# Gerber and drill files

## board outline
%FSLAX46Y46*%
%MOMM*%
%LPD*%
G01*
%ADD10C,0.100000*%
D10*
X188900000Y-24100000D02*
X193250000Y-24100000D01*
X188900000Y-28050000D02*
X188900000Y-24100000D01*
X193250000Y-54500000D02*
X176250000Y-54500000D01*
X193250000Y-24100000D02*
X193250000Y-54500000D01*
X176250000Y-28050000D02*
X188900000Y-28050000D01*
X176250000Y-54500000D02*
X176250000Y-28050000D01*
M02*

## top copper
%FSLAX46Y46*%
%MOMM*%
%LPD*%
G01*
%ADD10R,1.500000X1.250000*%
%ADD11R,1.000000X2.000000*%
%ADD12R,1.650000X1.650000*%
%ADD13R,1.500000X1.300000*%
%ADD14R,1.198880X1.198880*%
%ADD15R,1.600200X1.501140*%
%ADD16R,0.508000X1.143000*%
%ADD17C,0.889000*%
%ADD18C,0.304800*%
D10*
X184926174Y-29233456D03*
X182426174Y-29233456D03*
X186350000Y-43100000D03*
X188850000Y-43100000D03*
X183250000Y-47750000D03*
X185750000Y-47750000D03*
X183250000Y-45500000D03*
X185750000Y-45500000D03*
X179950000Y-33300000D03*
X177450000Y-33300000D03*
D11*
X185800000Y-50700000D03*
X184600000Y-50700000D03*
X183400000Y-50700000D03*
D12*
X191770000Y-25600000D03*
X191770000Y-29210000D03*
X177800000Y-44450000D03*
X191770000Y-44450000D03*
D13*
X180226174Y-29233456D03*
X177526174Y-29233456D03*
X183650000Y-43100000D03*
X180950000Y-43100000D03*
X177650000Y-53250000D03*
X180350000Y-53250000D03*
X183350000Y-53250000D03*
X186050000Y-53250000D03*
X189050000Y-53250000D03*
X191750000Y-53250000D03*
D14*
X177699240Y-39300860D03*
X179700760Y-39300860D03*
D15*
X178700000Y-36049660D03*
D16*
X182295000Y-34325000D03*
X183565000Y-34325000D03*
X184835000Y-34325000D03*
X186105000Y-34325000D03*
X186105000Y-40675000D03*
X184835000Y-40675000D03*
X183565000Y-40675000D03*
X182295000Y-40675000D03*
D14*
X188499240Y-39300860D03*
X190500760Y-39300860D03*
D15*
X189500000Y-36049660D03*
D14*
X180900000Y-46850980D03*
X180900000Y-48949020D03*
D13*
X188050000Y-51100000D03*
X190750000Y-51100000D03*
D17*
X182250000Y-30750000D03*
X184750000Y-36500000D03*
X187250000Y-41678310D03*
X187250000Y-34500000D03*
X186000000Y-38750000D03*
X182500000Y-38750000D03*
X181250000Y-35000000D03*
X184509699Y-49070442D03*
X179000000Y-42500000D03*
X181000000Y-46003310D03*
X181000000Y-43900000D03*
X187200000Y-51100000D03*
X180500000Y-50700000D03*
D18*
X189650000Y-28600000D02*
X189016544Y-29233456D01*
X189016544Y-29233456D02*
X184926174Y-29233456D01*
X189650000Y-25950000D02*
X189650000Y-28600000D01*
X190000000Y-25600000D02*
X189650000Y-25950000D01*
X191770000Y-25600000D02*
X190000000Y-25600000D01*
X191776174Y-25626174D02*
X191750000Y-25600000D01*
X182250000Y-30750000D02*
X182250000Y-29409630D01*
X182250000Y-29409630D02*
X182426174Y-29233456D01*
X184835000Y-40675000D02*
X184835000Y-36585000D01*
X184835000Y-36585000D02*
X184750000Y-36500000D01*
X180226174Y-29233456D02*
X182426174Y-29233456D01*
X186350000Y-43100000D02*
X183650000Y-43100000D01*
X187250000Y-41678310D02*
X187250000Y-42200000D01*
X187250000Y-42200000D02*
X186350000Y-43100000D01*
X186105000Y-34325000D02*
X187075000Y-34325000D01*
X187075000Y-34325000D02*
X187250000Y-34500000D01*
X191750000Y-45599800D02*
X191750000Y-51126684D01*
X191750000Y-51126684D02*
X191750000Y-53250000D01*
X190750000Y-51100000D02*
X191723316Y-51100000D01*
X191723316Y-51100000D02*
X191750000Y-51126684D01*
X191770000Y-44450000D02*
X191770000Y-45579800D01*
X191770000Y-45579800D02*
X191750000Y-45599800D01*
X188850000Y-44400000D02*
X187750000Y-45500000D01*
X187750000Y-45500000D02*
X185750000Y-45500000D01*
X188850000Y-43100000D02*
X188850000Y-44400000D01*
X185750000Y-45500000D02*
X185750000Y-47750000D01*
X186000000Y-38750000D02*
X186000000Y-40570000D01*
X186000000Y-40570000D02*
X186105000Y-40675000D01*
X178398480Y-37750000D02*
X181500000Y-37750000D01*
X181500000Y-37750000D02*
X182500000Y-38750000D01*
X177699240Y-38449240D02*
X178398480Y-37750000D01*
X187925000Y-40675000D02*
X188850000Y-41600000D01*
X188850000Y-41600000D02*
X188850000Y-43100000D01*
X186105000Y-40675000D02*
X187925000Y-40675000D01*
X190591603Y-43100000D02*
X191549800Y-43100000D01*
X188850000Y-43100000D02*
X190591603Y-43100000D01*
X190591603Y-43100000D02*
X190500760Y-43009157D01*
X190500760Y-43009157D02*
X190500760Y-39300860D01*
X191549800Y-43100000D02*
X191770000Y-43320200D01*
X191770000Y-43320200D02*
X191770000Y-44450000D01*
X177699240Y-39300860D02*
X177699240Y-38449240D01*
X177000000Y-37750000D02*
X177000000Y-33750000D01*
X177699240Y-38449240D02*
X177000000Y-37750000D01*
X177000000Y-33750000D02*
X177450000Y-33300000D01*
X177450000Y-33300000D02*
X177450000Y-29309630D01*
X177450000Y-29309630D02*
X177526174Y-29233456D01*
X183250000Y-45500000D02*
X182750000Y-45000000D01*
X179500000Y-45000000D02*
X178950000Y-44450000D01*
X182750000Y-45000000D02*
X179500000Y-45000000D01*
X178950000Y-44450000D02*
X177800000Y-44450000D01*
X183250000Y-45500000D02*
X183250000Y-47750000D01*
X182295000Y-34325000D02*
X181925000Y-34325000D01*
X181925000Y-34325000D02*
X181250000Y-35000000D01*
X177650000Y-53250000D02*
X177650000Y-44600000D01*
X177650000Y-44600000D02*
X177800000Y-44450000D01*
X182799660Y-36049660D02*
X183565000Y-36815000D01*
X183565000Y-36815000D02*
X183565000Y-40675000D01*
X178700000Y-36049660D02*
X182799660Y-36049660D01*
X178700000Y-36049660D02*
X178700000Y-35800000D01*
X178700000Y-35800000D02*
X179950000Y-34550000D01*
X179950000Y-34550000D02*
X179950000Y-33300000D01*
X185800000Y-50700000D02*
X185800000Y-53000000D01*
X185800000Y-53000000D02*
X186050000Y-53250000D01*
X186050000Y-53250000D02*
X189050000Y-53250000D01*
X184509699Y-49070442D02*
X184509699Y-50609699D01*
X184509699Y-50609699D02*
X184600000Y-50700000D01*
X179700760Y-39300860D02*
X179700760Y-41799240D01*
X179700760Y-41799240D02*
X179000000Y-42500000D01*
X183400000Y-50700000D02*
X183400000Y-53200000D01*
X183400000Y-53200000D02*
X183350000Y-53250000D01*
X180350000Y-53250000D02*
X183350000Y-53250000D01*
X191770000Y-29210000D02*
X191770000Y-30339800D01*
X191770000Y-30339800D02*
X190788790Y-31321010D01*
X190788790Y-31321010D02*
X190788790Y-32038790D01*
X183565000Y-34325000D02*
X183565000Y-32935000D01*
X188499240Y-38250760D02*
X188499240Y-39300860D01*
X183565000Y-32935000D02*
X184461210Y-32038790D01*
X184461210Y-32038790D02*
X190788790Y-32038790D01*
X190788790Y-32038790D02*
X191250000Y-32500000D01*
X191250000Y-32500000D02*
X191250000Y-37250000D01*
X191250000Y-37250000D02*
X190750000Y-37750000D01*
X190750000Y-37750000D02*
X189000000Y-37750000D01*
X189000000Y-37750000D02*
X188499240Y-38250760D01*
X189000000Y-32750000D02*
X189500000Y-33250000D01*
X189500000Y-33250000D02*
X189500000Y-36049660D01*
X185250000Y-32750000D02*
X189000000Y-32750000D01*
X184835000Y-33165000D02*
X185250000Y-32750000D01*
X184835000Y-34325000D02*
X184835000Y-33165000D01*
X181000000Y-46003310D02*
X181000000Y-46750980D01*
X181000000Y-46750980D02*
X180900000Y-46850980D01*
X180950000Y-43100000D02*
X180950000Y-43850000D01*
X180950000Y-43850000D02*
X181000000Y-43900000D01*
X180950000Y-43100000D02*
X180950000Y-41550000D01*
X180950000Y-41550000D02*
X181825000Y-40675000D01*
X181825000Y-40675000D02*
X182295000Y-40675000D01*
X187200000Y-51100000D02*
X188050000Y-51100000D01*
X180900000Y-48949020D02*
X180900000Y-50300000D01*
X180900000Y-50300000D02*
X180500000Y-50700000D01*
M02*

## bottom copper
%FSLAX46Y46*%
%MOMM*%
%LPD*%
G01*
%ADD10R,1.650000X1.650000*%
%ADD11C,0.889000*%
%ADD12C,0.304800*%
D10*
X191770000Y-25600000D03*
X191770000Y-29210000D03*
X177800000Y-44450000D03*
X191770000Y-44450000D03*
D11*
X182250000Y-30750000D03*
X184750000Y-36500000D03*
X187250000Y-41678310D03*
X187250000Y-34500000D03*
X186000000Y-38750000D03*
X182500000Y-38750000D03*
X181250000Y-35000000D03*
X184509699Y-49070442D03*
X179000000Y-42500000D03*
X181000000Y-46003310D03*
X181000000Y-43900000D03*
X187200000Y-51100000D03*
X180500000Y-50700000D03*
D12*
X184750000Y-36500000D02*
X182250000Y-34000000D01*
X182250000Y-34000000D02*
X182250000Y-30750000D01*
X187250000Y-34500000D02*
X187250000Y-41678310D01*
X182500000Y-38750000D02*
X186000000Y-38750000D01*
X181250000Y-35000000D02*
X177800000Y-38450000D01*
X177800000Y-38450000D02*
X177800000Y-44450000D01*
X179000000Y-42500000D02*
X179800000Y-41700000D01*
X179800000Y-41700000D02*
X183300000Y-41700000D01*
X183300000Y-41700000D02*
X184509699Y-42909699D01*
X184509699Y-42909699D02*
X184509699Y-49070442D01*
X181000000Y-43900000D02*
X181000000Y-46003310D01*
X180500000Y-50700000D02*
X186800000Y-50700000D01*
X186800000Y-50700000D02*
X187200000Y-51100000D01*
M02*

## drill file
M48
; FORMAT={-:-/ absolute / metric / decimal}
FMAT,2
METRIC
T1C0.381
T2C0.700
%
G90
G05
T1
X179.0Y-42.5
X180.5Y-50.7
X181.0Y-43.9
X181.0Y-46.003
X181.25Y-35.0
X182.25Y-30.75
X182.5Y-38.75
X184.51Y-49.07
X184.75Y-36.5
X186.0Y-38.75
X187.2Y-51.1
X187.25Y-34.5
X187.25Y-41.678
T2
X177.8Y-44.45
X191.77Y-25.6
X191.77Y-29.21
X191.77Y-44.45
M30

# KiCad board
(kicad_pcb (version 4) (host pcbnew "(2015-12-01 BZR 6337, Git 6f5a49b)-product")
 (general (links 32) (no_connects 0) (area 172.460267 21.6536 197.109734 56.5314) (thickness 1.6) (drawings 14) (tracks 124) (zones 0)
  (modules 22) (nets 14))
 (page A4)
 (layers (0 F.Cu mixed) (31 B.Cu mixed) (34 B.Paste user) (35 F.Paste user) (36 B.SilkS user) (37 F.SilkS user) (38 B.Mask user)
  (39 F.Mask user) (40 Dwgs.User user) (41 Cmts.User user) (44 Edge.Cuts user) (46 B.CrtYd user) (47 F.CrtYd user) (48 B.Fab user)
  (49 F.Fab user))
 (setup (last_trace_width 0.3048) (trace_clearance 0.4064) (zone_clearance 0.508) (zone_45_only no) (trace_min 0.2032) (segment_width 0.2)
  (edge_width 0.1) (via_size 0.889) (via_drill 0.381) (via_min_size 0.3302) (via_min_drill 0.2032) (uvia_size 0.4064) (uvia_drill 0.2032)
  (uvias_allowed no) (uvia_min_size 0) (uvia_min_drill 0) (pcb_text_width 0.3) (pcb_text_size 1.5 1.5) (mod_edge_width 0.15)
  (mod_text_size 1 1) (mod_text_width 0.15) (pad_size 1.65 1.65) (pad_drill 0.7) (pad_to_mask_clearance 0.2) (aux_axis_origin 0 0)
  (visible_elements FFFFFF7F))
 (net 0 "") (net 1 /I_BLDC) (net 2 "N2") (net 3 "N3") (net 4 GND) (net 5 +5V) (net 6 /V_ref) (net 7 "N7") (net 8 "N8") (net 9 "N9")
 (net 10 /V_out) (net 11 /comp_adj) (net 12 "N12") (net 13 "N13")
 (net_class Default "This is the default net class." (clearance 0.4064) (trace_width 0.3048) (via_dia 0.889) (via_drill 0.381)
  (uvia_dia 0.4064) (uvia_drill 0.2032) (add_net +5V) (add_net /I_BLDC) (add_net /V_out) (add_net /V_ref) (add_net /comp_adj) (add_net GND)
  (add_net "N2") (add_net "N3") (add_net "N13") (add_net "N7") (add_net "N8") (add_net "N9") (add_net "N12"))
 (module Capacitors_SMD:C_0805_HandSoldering (layer F.Cu) (at 183.676174 29.233456 180)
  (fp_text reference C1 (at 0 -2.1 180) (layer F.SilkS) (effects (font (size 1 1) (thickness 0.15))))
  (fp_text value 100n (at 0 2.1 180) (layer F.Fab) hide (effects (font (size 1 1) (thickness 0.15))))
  (pad 1 smd rect (at -1.25 0 180) (size 1.5 1.25) (layers F.Cu F.Paste F.Mask) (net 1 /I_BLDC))
  (pad 2 smd rect (at 1.25 0 180) (size 1.5 1.25) (layers F.Cu F.Paste F.Mask) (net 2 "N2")))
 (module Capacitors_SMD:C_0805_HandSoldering (layer F.Cu) (at 187.6 43.1)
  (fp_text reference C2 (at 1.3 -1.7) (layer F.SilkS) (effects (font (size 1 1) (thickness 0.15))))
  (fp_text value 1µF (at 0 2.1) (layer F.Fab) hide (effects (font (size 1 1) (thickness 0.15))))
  (pad 1 smd rect (at -1.25 0) (size 1.5 1.25) (layers F.Cu F.Paste F.Mask) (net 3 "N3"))
  (pad 2 smd rect (at 1.25 0) (size 1.5 1.25) (layers F.Cu F.Paste F.Mask) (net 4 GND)))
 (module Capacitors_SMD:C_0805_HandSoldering (layer F.Cu) (at 184.5 47.75)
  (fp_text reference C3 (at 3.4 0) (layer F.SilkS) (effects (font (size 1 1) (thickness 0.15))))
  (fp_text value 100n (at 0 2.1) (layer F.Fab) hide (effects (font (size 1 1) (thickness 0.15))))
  (pad 1 smd rect (at -1.25 0) (size 1.5 1.25) (layers F.Cu F.Paste F.Mask) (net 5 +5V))
  (pad 2 smd rect (at 1.25 0) (size 1.5 1.25) (layers F.Cu F.Paste F.Mask) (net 4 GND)))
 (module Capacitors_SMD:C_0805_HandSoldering (layer F.Cu) (at 184.5 45.5)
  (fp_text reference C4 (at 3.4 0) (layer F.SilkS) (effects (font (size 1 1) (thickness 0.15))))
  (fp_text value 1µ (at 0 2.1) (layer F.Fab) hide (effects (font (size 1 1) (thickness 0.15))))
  (pad 1 smd rect (at -1.25 0) (size 1.5 1.25) (layers F.Cu F.Paste F.Mask) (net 5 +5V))
  (pad 2 smd rect (at 1.25 0) (size 1.5 1.25) (layers F.Cu F.Paste F.Mask) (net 4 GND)))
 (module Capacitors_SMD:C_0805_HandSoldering (layer F.Cu) (at 178.7 33.3 180)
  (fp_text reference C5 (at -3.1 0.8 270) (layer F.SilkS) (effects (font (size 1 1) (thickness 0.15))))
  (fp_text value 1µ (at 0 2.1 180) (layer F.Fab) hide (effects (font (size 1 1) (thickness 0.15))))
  (pad 1 smd rect (at -1.25 0 180) (size 1.5 1.25) (layers F.Cu F.Paste F.Mask) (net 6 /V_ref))
  (pad 2 smd rect (at 1.25 0 180) (size 1.5 1.25) (layers F.Cu F.Paste F.Mask) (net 4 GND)))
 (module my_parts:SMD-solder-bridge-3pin (layer F.Cu) (at 184.6 50.7 180) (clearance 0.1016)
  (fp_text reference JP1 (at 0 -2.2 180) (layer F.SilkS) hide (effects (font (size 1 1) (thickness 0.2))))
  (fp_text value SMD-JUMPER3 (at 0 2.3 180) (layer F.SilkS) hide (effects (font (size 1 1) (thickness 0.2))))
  (pad 1 smd rect (at -1.2 0 180) (size 1 2) (layers F.Cu F.Mask) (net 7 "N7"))
  (pad 2 smd rect (at 0 0 180) (size 1 2) (layers F.Cu F.Mask) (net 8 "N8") (solder_mask_margin 0.3))
  (pad 3 smd rect (at 1.2 0 180) (size 1 2) (layers F.Cu F.Mask) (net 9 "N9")))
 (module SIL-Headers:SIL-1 (layer F.Cu) (at 191.77 25.6)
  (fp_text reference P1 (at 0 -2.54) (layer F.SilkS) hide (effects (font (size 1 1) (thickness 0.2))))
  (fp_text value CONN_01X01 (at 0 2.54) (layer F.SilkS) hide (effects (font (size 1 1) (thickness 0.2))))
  (pad 1 thru_hole rect (at 0 0) (size 1.65 1.65) (drill 0.7) (layers *.Cu *.Mask) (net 1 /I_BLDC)))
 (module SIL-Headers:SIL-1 (layer F.Cu) (at 191.77 29.21)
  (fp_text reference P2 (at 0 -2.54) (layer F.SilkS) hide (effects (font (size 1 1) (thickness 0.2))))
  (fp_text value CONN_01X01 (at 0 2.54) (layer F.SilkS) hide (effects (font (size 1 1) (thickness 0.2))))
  (pad 1 thru_hole rect (at 0 0) (size 1.65 1.65) (drill 0.7) (layers *.Cu *.Mask) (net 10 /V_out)))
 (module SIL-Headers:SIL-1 (layer F.Cu) (at 177.8 44.45)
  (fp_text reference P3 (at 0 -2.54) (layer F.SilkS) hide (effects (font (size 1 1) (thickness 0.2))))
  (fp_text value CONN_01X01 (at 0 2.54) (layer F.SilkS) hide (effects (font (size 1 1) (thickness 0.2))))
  (pad 1 thru_hole rect (at 0 0) (size 1.65 1.65) (drill 0.7) (layers *.Cu *.Mask) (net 5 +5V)))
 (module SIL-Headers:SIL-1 (layer F.Cu) (at 191.77 44.45)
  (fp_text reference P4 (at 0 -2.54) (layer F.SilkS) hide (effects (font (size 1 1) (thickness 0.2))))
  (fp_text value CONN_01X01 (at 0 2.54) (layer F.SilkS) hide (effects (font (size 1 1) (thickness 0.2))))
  (pad 1 thru_hole rect (at 0 0) (size 1.65 1.65) (drill 0.7) (layers *.Cu *.Mask) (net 4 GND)))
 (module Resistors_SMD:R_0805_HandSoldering (layer F.Cu) (at 178.876174 29.233456 180)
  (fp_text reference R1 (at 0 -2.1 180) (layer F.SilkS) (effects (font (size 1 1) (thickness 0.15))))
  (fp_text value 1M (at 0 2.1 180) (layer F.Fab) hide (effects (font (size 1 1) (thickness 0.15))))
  (pad 1 smd rect (at -1.35 0 180) (size 1.5 1.3) (layers F.Cu F.Paste F.Mask) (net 2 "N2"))
  (pad 2 smd rect (at 1.35 0 180) (size 1.5 1.3) (layers F.Cu F.Paste F.Mask) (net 4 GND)))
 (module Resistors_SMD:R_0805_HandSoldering (layer F.Cu) (at 182.3 43.1 180)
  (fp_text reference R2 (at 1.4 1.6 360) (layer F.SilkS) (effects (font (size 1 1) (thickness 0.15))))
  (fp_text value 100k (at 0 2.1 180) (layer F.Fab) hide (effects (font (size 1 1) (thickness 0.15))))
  (pad 1 smd rect (at -1.35 0 180) (size 1.5 1.3) (layers F.Cu F.Paste F.Mask) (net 3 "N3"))
  (pad 2 smd rect (at 1.35 0 180) (size 1.5 1.3) (layers F.Cu F.Paste F.Mask) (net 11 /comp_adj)))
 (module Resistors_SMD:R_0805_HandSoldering (layer F.Cu) (at 179 53.25)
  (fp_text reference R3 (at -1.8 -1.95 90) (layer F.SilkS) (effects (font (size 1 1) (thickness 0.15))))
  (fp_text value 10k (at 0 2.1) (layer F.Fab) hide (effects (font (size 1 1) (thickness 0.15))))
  (pad 1 smd rect (at -1.35 0) (size 1.5 1.3) (layers F.Cu F.Paste F.Mask) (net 5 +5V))
  (pad 2 smd rect (at 1.35 0) (size 1.5 1.3) (layers F.Cu F.Paste F.Mask) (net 9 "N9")))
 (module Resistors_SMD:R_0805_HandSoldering (layer F.Cu) (at 184.7 53.25)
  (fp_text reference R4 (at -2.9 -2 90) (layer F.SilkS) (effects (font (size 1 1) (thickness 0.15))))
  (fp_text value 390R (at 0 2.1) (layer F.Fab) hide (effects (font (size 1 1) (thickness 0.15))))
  (pad 1 smd rect (at -1.35 0) (size 1.5 1.3) (layers F.Cu F.Paste F.Mask) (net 9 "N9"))
  (pad 2 smd rect (at 1.35 0) (size 1.5 1.3) (layers F.Cu F.Paste F.Mask) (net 7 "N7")))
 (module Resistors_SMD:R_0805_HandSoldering (layer F.Cu) (at 190.4 53.25)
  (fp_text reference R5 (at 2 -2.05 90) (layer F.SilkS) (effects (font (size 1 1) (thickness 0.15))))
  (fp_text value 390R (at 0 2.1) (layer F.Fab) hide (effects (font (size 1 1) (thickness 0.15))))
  (pad 1 smd rect (at -1.35 0) (size 1.5 1.3) (layers F.Cu F.Paste F.Mask) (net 7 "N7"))
  (pad 2 smd rect (at 1.35 0) (size 1.5 1.3) (layers F.Cu F.Paste F.Mask) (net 4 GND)))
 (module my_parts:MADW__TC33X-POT (layer F.Cu) (at 178.7 37.5)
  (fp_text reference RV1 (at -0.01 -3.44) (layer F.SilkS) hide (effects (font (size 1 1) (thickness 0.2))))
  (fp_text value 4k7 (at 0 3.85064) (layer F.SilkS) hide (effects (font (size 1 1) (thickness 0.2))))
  (pad 1 smd rect (at -1.00076 1.80086) (size 1.19888 1.19888) (layers F.Cu F.Paste F.Mask) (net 4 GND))
  (pad 3 smd rect (at 1.00076 1.80086) (size 1.19888 1.19888) (layers F.Cu F.Paste F.Mask) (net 8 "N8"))
  (pad 2 smd rect (at 0 -1.45034) (size 1.6002 1.50114) (layers F.Cu F.Paste F.Mask) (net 6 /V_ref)))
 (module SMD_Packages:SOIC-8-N (layer F.Cu) (at 184.2 37.5)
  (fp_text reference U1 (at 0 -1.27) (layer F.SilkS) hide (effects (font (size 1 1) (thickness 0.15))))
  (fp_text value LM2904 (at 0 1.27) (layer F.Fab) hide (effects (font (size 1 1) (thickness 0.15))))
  (pad 8 smd rect (at -1.905 -3.175) (size 0.508 1.143) (layers F.Cu F.Paste F.Mask) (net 5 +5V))
  (pad 7 smd rect (at -0.635 -3.175) (size 0.508 1.143) (layers F.Cu F.Paste F.Mask) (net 10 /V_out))
  (pad 6 smd rect (at 0.635 -3.175) (size 0.508 1.143) (layers F.Cu F.Paste F.Mask) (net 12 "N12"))
  (pad 5 smd rect (at 1.905 -3.175) (size 0.508 1.143) (layers F.Cu F.Paste F.Mask) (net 3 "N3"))
  (pad 4 smd rect (at 1.905 3.175) (size 0.508 1.143) (layers F.Cu F.Paste F.Mask) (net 4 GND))
  (pad 3 smd rect (at 0.635 3.175) (size 0.508 1.143) (layers F.Cu F.Paste F.Mask) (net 2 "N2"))
  (pad 2 smd rect (at -0.635 3.175) (size 0.508 1.143) (layers F.Cu F.Paste F.Mask) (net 6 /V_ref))
  (pad 1 smd rect (at -1.905 3.175) (size 0.508 1.143) (layers F.Cu F.Paste F.Mask) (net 11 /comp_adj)))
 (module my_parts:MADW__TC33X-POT (layer F.Cu) (at 189.5 37.5)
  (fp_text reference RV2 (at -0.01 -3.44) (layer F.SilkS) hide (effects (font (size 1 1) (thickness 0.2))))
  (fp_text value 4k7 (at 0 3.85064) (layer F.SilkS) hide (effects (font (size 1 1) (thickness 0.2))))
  (pad 1 smd rect (at -1.00076 1.80086) (size 1.19888 1.19888) (layers F.Cu F.Paste F.Mask) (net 10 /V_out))
  (pad 3 smd rect (at 1.00076 1.80086) (size 1.19888 1.19888) (layers F.Cu F.Paste F.Mask) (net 4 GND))
  (pad 2 smd rect (at 0 -1.45034) (size 1.6002 1.50114) (layers F.Cu F.Paste F.Mask) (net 12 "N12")))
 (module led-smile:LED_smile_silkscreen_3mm (layer F.Cu) (at 186.85 31.85)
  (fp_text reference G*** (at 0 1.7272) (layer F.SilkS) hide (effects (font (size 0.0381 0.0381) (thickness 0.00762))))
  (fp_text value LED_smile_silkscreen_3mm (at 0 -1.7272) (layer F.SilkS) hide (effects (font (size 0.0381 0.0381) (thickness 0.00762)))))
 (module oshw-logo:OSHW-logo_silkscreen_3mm (layer F.Cu) (at 191.7 41.45)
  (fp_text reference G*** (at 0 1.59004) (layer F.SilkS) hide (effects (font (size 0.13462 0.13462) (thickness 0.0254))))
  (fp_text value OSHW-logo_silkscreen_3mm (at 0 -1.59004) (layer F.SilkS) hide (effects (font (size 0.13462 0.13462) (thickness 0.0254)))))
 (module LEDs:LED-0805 (layer F.Cu) (at 180.9 47.9 90)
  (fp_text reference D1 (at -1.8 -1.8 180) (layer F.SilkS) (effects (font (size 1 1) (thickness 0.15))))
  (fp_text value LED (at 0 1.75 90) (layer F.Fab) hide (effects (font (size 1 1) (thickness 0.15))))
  (pad 2 smd rect (at 1.04902 0 270) (size 1.19888 1.19888) (layers F.Cu F.Paste F.Mask) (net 11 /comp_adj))
  (pad 1 smd rect (at -1.04902 0 270) (size 1.19888 1.19888) (layers F.Cu F.Paste F.Mask) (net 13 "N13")))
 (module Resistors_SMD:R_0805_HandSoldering (layer F.Cu) (at 189.4 51.1)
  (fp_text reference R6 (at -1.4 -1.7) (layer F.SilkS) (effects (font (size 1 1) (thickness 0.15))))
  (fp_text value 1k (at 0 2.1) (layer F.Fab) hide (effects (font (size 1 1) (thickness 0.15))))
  (pad 1 smd rect (at -1.35 0) (size 1.5 1.3) (layers F.Cu F.Paste F.Mask) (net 13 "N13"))
  (pad 2 smd rect (at 1.35 0) (size 1.5 1.3) (layers F.Cu F.Paste F.Mask) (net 4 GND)))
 (gr_line (start 188.9 24.1) (end 193.25 24.1) (layer Edge.Cuts) (width 0.1))
 (gr_line (start 188.9 28.05) (end 188.9 24.1) (layer Edge.Cuts) (width 0.1))
 (gr_line (start 193.25 54.5) (end 176.25 54.5) (layer Edge.Cuts) (width 0.1))
 (gr_line (start 193.25 24.1) (end 193.25 54.5) (layer Edge.Cuts) (width 0.1))
 (gr_line (start 176.25 28.05) (end 188.9 28.05) (layer Edge.Cuts) (width 0.1))
 (gr_line (start 176.25 54.5) (end 176.25 28.05) (layer Edge.Cuts) (width 0.1))
 (segment (start 189.65 28.6) (end 189.016544 29.233456) (width 0.3048) (layer F.Cu) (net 1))
 (segment (start 189.016544 29.233456) (end 184.926174 29.233456) (width 0.3048) (layer F.Cu) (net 1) (status 20))
 (segment (start 189.65 25.95) (end 189.65 28.6) (width 0.3048) (layer F.Cu) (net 1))
 (segment (start 190 25.6) (end 189.65 25.95) (width 0.3048) (layer F.Cu) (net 1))
 (segment (start 191.77 25.6) (end 190 25.6) (width 0.3048) (layer F.Cu) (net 1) (status 10))
 (segment (start 191.776174 25.626174) (end 191.75 25.6) (width 0.3048) (layer F.Cu) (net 1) (status 30))
 (segment (start 182.25 30.75) (end 182.25 29.40963) (width 0.3048) (layer F.Cu) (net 2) (status 20))
 (segment (start 182.25 29.40963) (end 182.426174 29.233456) (width 0.3048) (layer F.Cu) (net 2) (status 30))
 (segment (start 184.75 36.5) (end 182.25 34) (width 0.3048) (layer B.Cu) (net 2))
 (segment (start 182.25 34) (end 182.25 30.75) (width 0.3048) (layer B.Cu) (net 2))
 (via (at 182.25 30.75) (size 0.889) (drill 0.381) (layers F.Cu B.Cu) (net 2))
 (segment (start 184.835 40.675) (end 184.835 36.585) (width 0.3048) (layer F.Cu) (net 2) (status 10))
 (segment (start 184.835 36.585) (end 184.75 36.5) (width 0.3048) (layer F.Cu) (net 2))
 (via (at 184.75 36.5) (size 0.889) (drill 0.381) (layers F.Cu B.Cu) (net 2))
 (segment (start 180.226174 29.233456) (end 182.426174 29.233456) (width 0.3048) (layer F.Cu) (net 2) (status 30))
 (segment (start 186.35 43.1) (end 183.65 43.1) (width 0.3048) (layer F.Cu) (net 3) (status 30))
 (segment (start 187.25 41.67831) (end 187.25 42.2) (width 0.3048) (layer F.Cu) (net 3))
 (segment (start 187.25 42.2) (end 186.35 43.1) (width 0.3048) (layer F.Cu) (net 3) (status 20))
 (segment (start 187.25 34.5) (end 187.25 41.67831) (width 0.3048) (layer B.Cu) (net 3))
 (via (at 187.25 41.67831) (size 0.889) (drill 0.381) (layers F.Cu B.Cu) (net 3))
 (segment (start 186.105 34.325) (end 187.075 34.325) (width 0.3048) (layer F.Cu) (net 3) (status 10))
 (segment (start 187.075 34.325) (end 187.25 34.5) (width 0.3048) (layer F.Cu) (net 3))
 (via (at 187.25 34.5) (size 0.889) (drill 0.381) (layers F.Cu B.Cu) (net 3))
 (segment (start 191.75 45.5998) (end 191.75 51.126684) (width 0.3048) (layer F.Cu) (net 4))
 (segment (start 191.75 51.126684) (end 191.75 53.25) (width 0.3048) (layer F.Cu) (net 4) (status 20))
 (segment (start 190.75 51.1) (end 191.723316 51.1) (width 0.3048) (layer F.Cu) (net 4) (status 10))
 (segment (start 191.723316 51.1) (end 191.75 51.126684) (width 0.3048) (layer F.Cu) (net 4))
 (segment (start 191.77 44.45) (end 191.77 45.5798) (width 0.3048) (layer F.Cu) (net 4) (status 10))
 (segment (start 191.77 45.5798) (end 191.75 45.5998) (width 0.3048) (layer F.Cu) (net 4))
 (segment (start 188.85 44.4) (end 187.75 45.5) (width 0.3048) (layer F.Cu) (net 4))
 (segment (start 187.75 45.5) (end 185.75 45.5) (width 0.3048) (layer F.Cu) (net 4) (status 20))
 (segment (start 188.85 43.1) (end 188.85 44.4) (width 0.3048) (layer F.Cu) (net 4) (status 10))
 (segment (start 185.75 45.5) (end 185.75 47.75) (width 0.3048) (layer F.Cu) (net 4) (status 30))
 (segment (start 186 38.75) (end 186 40.57) (width 0.3048) (layer F.Cu) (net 4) (status 20))
 (segment (start 186 40.57) (end 186.105 40.675) (width 0.3048) (layer F.Cu) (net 4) (status 30))
 (segment (start 182.5 38.75) (end 186 38.75) (width 0.3048) (layer B.Cu) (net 4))
 (via (at 186 38.75) (size 0.889) (drill 0.381) (layers F.Cu B.Cu) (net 4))
 (segment (start 178.39848 37.75) (end 181.5 37.75) (width 0.3048) (layer F.Cu) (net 4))
 (segment (start 181.5 37.75) (end 182.5 38.75) (width 0.3048) (layer F.Cu) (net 4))
 (segment (start 177.69924 38.44924) (end 178.39848 37.75) (width 0.3048) (layer F.Cu) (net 4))
 (via (at 182.5 38.75) (size 0.889) (drill 0.381) (layers F.Cu B.Cu) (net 4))
 (segment (start 187.925 40.675) (end 188.85 41.6) (width 0.3048) (layer F.Cu) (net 4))
 (segment (start 188.85 41.6) (end 188.85 43.1) (width 0.3048) (layer F.Cu) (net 4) (status 20))
 (segment (start 186.105 40.675) (end 187.925 40.675) (width 0.3048) (layer F.Cu) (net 4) (status 10))
 (segment (start 190.591603 43.1) (end 191.5498 43.1) (width 0.3048) (layer F.Cu) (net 4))
 (segment (start 188.85 43.1) (end 190.591603 43.1) (width 0.3048) (layer F.Cu) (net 4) (status 10))
 (segment (start 190.591603 43.1) (end 190.50076 43.009157) (width 0.3048) (layer F.Cu) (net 4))
 (segment (start 190.50076 43.009157) (end 190.50076 39.30086) (width 0.3048) (layer F.Cu) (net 4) (status 20))
 (segment (start 191.5498 43.1) (end 191.77 43.3202) (width 0.3048) (layer F.Cu) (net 4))
 (segment (start 191.77 43.3202) (end 191.77 44.45) (width 0.3048) (layer F.Cu) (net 4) (status 20))
 (segment (start 177.69924 39.30086) (end 177.69924 38.44924) (width 0.3048) (layer F.Cu) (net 4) (status 10))
 (segment (start 177 37.75) (end 177 33.75) (width 0.3048) (layer F.Cu) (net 4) (status 20))
 (segment (start 177.69924 38.44924) (end 177 37.75) (width 0.3048) (layer F.Cu) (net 4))
 (segment (start 177 33.75) (end 177.45 33.3) (width 0.3048) (layer F.Cu) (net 4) (status 30))
 (segment (start 177.45 33.3) (end 177.45 29.30963) (width 0.3048) (layer F.Cu) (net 4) (status 30))
 (segment (start 177.45 29.30963) (end 177.526174 29.233456) (width 0.3048) (layer F.Cu) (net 4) (status 30))
 (segment (start 183.25 45.5) (end 182.75 45) (width 0.3048) (layer F.Cu) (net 5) (status 30))
 (segment (start 179.5 45) (end 178.95 44.45) (width 0.3048) (layer F.Cu) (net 5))
 (segment (start 182.75 45) (end 179.5 45) (width 0.3048) (layer F.Cu) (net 5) (status 10))
 (segment (start 178.95 44.45) (end 177.8 44.45) (width 0.3048) (layer F.Cu) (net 5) (status 20))
 (segment (start 183.25 45.5) (end 183.25 47.75) (width 0.3048) (layer F.Cu) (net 5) (status 30))
 (segment (start 181.25 35) (end 177.8 38.45) (width 0.3048) (layer B.Cu) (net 5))
 (segment (start 177.8 38.45) (end 177.8 44.45) (width 0.3048) (layer B.Cu) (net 5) (status 20))
 (segment (start 182.295 34.325) (end 181.925 34.325) (width 0.3048) (layer F.Cu) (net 5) (status 10))
 (via (at 181.25 35) (size 0.889) (drill 0.381) (layers F.Cu B.Cu) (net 5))
 (segment (start 181.925 34.325) (end 181.25 35) (width 0.3048) (layer F.Cu) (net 5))
 (segment (start 177.65 53.25) (end 177.65 44.6) (width 0.3048) (layer F.Cu) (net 5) (status 30))
 (segment (start 177.65 44.6) (end 177.8 44.45) (width 0.3048) (layer F.Cu) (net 5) (status 30))
 (segment (start 182.79966 36.04966) (end 183.565 36.815) (width 0.3048) (layer F.Cu) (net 6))
 (segment (start 183.565 36.815) (end 183.565 40.675) (width 0.3048) (layer F.Cu) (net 6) (status 20))
 (segment (start 178.7 36.04966) (end 182.79966 36.04966) (width 0.3048) (layer F.Cu) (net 6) (status 10))
 (segment (start 178.7 36.04966) (end 178.7 35.8) (width 0.3048) (layer F.Cu) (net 6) (status 30))
 (segment (start 178.7 35.8) (end 179.95 34.55) (width 0.3048) (layer F.Cu) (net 6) (status 10))
 (segment (start 179.95 34.55) (end 179.95 33.3) (width 0.3048) (layer F.Cu) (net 6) (status 20))
 (segment (start 185.8 50.7) (end 185.8 53) (width 0.3048) (layer F.Cu) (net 7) (status 30))
 (segment (start 185.8 53) (end 186.05 53.25) (width 0.3048) (layer F.Cu) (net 7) (status 30))
 (segment (start 186.05 53.25) (end 189.05 53.25) (width 0.3048) (layer F.Cu) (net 7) (status 30))
 (segment (start 179 42.5) (end 179.8 41.7) (width 0.3048) (layer B.Cu) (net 8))
 (segment (start 179.8 41.7) (end 183.3 41.7) (width 0.3048) (layer B.Cu) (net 8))
 (segment (start 183.3 41.7) (end 184.509699 42.909699) (width 0.3048) (layer B.Cu) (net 8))
 (segment (start 184.509699 42.909699) (end 184.509699 49.070442) (width 0.3048) (layer B.Cu) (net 8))
 (segment (start 184.509699 49.070442) (end 184.509699 50.609699) (width 0.3048) (layer F.Cu) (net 8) (status 20))
 (segment (start 184.509699 50.609699) (end 184.6 50.7) (width 0.3048) (layer F.Cu) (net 8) (status 30))
 (via (at 184.509699 49.070442) (size 0.889) (drill 0.381) (layers F.Cu B.Cu) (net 8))
 (segment (start 179.70076 39.30086) (end 179.70076 41.79924) (width 0.3048) (layer F.Cu) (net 8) (status 10))
 (segment (start 179.70076 41.79924) (end 179 42.5) (width 0.3048) (layer F.Cu) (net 8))
 (via (at 179 42.5) (size 0.889) (drill 0.381) (layers F.Cu B.Cu) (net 8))
 (segment (start 183.4 50.7) (end 183.4 53.2) (width 0.3048) (layer F.Cu) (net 9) (status 30))
 (segment (start 183.4 53.2) (end 183.35 53.25) (width 0.3048) (layer F.Cu) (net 9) (status 30))
 (segment (start 180.35 53.25) (end 183.35 53.25) (width 0.3048) (layer F.Cu) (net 9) (status 30))
 (segment (start 191.77 29.21) (end 191.77 30.3398) (width 0.3048) (layer F.Cu) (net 10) (status 10))
 (segment (start 191.77 30.3398) (end 190.78879 31.32101) (width 0.3048) (layer F.Cu) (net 10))
 (segment (start 190.78879 31.32101) (end 190.78879 32.03879) (width 0.3048) (layer F.Cu) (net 10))
 (segment (start 183.565 34.325) (end 183.565 32.935) (width 0.3048) (layer F.Cu) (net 10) (status 10))
 (segment (start 188.49924 38.25076) (end 188.49924 39.30086) (width 0.3048) (layer F.Cu) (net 10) (status 20))
 (segment (start 183.565 32.935) (end 184.46121 32.03879) (width 0.3048) (layer F.Cu) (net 10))
 (segment (start 184.46121 32.03879) (end 190.78879 32.03879) (width 0.3048) (layer F.Cu) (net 10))
 (segment (start 190.78879 32.03879) (end 191.25 32.5) (width 0.3048) (layer F.Cu) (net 10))
 (segment (start 191.25 32.5) (end 191.25 37.25) (width 0.3048) (layer F.Cu) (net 10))
 (segment (start 191.25 37.25) (end 190.75 37.75) (width 0.3048) (layer F.Cu) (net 10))
 (segment (start 190.75 37.75) (end 189 37.75) (width 0.3048) (layer F.Cu) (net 10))
 (segment (start 189 37.75) (end 188.49924 38.25076) (width 0.3048) (layer F.Cu) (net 10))
 (segment (start 189 32.75) (end 189.5 33.25) (width 0.3048) (layer F.Cu) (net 12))
 (segment (start 189.5 33.25) (end 189.5 36.04966) (width 0.3048) (layer F.Cu) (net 12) (status 20))
 (segment (start 185.25 32.75) (end 189 32.75) (width 0.3048) (layer F.Cu) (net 12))
 (segment (start 184.835 33.165) (end 185.25 32.75) (width 0.3048) (layer F.Cu) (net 12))
 (segment (start 184.835 34.325) (end 184.835 33.165) (width 0.3048) (layer F.Cu) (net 12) (status 10))
 (segment (start 181 46.00331) (end 181 46.75098) (width 0.3048) (layer F.Cu) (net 11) (status 20))
 (segment (start 181 46.75098) (end 180.9 46.85098) (width 0.3048) (layer F.Cu) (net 11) (status 30))
 (segment (start 181 43.9) (end 181 46.00331) (width 0.3048) (layer B.Cu) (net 11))
 (via (at 181 46.00331) (size 0.889) (drill 0.381) (layers F.Cu B.Cu) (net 11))
 (segment (start 180.95 43.1) (end 180.95 43.85) (width 0.3048) (layer F.Cu) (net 11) (status 10))
 (segment (start 180.95 43.85) (end 181 43.9) (width 0.3048) (layer F.Cu) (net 11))
 (via (at 181 43.9) (size 0.889) (drill 0.381) (layers F.Cu B.Cu) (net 11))
 (segment (start 180.95 43.1) (end 180.95 41.55) (width 0.3048) (layer F.Cu) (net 11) (status 10))
 (segment (start 180.95 41.55) (end 181.825 40.675) (width 0.3048) (layer F.Cu) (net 11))
 (segment (start 181.825 40.675) (end 182.295 40.675) (width 0.3048) (layer F.Cu) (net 11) (status 20))
 (segment (start 187.2 51.1) (end 188.05 51.1) (width 0.3048) (layer F.Cu) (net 13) (status 20))
 (segment (start 180.5 50.7) (end 186.8 50.7) (width 0.3048) (layer B.Cu) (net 13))
 (segment (start 186.8 50.7) (end 187.2 51.1) (width 0.3048) (layer B.Cu) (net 13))
 (via (at 187.2 51.1) (size 0.889) (drill 0.381) (layers F.Cu B.Cu) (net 13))
 (segment (start 180.9 48.94902) (end 180.9 50.3) (width 0.3048) (layer F.Cu) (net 13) (status 10))
 (segment (start 180.9 50.3) (end 180.5 50.7) (width 0.3048) (layer F.Cu) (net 13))
 (via (at 180.5 50.7) (size 0.889) (drill 0.381) (layers F.Cu B.Cu) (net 13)))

